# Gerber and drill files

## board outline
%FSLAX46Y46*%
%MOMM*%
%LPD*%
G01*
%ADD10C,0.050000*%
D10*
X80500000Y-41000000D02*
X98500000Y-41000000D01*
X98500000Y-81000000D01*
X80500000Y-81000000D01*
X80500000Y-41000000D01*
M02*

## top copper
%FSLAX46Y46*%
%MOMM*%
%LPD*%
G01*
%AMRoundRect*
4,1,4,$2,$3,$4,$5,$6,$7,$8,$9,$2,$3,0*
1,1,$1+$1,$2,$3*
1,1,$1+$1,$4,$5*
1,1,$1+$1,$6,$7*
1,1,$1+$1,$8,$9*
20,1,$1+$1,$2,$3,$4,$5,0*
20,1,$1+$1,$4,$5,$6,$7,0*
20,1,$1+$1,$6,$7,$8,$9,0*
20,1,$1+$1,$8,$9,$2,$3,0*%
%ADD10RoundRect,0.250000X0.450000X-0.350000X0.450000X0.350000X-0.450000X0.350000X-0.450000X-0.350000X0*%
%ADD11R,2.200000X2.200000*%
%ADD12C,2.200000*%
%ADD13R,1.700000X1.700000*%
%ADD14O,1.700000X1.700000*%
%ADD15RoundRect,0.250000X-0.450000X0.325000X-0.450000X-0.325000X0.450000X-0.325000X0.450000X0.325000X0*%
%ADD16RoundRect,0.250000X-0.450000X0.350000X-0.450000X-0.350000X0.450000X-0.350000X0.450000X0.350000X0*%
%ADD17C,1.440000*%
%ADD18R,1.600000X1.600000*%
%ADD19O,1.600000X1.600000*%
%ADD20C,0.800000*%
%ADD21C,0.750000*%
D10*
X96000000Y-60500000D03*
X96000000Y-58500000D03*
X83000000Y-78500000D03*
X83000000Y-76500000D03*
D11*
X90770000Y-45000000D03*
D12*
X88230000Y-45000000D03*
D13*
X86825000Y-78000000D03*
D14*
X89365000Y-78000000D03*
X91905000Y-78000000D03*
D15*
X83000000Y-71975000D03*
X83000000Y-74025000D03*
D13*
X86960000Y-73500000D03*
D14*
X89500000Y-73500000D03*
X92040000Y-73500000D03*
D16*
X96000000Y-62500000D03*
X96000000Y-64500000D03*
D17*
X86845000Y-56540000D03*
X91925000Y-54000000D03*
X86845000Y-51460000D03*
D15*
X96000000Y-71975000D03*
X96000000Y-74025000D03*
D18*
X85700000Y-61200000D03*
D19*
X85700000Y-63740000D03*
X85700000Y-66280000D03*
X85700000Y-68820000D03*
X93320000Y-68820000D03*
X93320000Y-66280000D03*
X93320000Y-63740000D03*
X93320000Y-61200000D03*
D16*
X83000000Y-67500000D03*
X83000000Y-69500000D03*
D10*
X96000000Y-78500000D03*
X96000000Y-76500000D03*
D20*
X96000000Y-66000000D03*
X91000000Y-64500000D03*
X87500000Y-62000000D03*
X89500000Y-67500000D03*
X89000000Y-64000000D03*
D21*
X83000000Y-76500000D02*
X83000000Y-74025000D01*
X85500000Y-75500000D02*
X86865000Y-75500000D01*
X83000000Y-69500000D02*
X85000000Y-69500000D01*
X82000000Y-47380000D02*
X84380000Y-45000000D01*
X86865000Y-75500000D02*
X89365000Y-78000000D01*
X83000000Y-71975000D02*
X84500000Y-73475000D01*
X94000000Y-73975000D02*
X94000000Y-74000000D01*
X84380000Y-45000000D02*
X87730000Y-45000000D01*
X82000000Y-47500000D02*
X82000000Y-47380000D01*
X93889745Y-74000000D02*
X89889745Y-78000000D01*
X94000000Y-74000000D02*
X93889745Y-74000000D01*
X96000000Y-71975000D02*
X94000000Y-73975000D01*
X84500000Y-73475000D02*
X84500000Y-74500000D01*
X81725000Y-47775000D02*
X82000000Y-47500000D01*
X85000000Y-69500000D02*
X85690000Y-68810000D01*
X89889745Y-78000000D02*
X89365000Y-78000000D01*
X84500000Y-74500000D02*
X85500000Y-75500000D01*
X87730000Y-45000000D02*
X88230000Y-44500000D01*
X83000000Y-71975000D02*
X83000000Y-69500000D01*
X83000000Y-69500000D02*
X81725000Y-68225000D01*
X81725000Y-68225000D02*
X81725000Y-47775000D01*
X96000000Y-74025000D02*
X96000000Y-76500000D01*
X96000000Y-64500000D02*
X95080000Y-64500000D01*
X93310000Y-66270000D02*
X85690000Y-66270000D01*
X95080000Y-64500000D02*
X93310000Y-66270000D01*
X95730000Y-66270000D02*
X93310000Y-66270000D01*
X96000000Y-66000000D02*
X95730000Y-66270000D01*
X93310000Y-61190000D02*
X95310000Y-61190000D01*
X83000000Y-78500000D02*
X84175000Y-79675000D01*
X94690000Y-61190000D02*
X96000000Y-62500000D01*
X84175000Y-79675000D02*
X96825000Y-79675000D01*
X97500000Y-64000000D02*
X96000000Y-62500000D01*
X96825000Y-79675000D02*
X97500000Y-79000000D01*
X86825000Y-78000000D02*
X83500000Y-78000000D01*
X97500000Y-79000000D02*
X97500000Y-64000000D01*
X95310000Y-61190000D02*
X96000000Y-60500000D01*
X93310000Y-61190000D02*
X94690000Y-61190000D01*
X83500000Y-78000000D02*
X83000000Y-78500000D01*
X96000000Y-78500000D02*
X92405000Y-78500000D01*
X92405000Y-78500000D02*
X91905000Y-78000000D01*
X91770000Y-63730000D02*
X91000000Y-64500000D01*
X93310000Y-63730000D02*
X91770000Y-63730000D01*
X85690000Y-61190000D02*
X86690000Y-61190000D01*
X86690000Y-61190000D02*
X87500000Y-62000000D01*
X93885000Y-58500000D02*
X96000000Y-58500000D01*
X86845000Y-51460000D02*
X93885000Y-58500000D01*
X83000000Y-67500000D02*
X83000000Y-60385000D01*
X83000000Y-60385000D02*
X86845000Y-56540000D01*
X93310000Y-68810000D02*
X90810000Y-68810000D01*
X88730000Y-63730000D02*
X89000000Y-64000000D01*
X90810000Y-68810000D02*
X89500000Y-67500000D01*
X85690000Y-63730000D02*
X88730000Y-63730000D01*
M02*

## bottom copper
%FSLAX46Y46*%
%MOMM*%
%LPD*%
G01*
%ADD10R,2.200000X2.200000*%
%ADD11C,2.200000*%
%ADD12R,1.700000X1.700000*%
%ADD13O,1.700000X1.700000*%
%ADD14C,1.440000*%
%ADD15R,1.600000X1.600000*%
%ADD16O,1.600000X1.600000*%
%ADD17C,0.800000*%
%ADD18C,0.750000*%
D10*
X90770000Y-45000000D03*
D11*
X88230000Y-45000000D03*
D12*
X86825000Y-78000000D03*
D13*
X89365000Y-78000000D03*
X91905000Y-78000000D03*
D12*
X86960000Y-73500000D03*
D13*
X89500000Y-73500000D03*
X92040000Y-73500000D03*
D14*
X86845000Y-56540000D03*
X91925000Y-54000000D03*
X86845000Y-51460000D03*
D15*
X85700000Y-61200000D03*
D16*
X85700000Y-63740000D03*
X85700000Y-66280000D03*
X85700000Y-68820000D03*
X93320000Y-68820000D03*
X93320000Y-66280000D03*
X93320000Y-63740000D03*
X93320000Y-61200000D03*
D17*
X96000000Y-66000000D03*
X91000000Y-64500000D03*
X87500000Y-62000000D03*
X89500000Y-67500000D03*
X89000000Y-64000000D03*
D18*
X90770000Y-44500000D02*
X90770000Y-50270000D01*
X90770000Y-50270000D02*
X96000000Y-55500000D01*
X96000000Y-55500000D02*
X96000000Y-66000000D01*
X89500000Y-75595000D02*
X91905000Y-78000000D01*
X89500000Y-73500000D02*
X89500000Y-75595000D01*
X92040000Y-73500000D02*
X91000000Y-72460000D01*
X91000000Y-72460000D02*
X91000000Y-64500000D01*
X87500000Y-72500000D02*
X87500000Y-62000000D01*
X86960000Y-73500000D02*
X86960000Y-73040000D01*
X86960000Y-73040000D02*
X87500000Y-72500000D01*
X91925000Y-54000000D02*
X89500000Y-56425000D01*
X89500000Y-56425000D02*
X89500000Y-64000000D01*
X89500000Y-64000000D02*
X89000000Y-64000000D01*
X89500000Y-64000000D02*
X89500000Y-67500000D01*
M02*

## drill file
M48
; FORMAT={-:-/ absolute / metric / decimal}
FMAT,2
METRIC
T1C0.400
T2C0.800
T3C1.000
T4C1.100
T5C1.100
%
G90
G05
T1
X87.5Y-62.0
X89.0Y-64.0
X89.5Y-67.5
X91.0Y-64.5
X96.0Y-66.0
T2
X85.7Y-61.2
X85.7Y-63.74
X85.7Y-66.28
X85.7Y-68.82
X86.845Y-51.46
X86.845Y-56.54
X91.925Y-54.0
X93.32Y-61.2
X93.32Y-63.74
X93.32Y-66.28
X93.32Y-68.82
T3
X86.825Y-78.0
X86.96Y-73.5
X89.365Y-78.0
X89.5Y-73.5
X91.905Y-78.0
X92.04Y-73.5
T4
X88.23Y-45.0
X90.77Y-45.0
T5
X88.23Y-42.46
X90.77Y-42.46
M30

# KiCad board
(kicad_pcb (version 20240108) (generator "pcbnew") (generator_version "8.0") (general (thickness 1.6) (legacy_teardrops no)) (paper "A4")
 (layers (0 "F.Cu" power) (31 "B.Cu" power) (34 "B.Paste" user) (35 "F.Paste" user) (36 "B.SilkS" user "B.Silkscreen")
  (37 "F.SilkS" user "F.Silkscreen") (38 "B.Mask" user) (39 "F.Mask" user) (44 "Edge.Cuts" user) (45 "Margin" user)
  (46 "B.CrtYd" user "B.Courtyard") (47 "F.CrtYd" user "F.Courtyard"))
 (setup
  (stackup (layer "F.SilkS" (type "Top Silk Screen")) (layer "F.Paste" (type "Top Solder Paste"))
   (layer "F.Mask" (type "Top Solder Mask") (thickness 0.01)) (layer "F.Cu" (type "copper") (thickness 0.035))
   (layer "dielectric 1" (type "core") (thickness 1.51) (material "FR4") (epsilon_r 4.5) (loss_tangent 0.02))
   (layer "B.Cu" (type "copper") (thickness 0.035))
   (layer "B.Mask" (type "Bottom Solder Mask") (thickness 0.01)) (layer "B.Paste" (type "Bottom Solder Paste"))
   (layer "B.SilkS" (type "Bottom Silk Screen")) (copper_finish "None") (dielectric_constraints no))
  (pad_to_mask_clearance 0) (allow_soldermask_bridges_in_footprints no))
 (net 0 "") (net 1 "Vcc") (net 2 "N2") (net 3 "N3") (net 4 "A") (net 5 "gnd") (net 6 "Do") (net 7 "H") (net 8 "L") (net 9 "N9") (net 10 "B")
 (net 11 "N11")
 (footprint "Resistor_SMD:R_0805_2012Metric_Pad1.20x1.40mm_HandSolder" (layer "F.Cu") (at 96 59.5 90)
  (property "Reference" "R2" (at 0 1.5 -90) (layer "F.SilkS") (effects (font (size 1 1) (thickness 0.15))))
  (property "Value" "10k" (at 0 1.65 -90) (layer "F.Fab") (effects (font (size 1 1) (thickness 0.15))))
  (pad "1" smd roundrect (at -1 0 90) (size 1.2 1.4) (layers "F.Cu" "F.Paste" "F.Mask") (roundrect_rratio 0.208333) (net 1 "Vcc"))
  (pad "2" smd roundrect (at 1 0 90) (size 1.2 1.4) (layers "F.Cu" "F.Paste" "F.Mask") (roundrect_rratio 0.208333) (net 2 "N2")))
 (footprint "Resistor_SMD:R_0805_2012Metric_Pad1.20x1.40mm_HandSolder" (layer "F.Cu") (at 83 77.5 90)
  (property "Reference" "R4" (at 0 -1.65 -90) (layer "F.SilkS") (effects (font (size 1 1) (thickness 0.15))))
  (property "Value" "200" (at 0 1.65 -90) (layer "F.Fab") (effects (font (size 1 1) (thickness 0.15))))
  (pad "1" smd roundrect (at -1 0 90) (size 1.2 1.4) (layers "F.Cu" "F.Paste" "F.Mask") (roundrect_rratio 0.208333) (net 1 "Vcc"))
  (pad "2" smd roundrect (at 1 0 90) (size 1.2 1.4) (layers "F.Cu" "F.Paste" "F.Mask") (roundrect_rratio 0.208333) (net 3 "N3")))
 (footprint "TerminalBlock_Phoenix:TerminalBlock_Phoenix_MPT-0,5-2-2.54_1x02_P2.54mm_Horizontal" (layer "F.Cu") (at 90.77 45 180)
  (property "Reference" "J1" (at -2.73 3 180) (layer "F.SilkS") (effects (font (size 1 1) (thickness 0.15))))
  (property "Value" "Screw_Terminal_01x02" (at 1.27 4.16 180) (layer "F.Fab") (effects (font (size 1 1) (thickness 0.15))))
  (pad "" np_thru_hole circle (at 0 2.54 180) (size 1.1 1.1) (drill 1.1) (layers "*.Cu" "*.Mask"))
  (pad "" np_thru_hole circle (at 2.54 2.54 180) (size 1.1 1.1) (drill 1.1) (layers "*.Cu" "*.Mask"))
  (pad "1" thru_hole rect (at 0 0 180) (size 2.2 2.2) (drill 1.1) (layers "*.Cu" "*.Mask") (remove_unused_layers no) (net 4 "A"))
  (pad "2" thru_hole circle (at 2.54 0 180) (size 2.2 2.2) (drill 1.1) (layers "*.Cu" "*.Mask") (remove_unused_layers no) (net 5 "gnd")))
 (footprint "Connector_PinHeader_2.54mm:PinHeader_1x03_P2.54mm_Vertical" (layer "F.Cu") (at 86.825 78 90)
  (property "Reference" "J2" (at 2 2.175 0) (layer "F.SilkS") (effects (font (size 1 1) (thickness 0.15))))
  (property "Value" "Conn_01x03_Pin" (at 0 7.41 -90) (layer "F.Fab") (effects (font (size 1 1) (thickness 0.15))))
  (pad "1" thru_hole rect (at 0 0 90) (size 1.7 1.7) (drill 1) (layers "*.Cu" "*.Mask") (remove_unused_layers no) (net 1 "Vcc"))
  (pad "2" thru_hole oval (at 0 2.54 90) (size 1.7 1.7) (drill 1) (layers "*.Cu" "*.Mask") (remove_unused_layers no) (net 5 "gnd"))
  (pad "3" thru_hole oval (at 0 5.08 90) (size 1.7 1.7) (drill 1) (layers "*.Cu" "*.Mask") (remove_unused_layers no) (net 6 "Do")))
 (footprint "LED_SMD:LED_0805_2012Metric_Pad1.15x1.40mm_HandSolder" (layer "F.Cu") (at 83 73 -90)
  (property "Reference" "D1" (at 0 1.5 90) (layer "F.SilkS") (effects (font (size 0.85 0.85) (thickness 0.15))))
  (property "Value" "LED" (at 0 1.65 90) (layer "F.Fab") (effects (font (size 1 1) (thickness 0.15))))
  (pad "1" smd roundrect (at -1.025 0 270) (size 1.15 1.4) (layers "F.Cu" "F.Paste" "F.Mask") (roundrect_rratio 0.217391) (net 5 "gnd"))
  (pad "2" smd roundrect (at 1.025 0 270) (size 1.15 1.4) (layers "F.Cu" "F.Paste" "F.Mask") (roundrect_rratio 0.217391) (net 3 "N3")))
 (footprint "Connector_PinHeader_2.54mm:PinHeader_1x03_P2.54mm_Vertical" (layer "F.Cu") (at 86.96 73.5 90)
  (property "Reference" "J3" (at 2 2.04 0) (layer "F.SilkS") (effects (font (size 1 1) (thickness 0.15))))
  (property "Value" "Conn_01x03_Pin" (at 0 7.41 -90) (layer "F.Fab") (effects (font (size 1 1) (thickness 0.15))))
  (pad "1" thru_hole rect (at 0 0 90) (size 1.7 1.7) (drill 1) (layers "*.Cu" "*.Mask") (remove_unused_layers no) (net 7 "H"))
  (pad "2" thru_hole oval (at 0 2.54 90) (size 1.7 1.7) (drill 1) (layers "*.Cu" "*.Mask") (remove_unused_layers no) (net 6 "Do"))
  (pad "3" thru_hole oval (at 0 5.08 90) (size 1.7 1.7) (drill 1) (layers "*.Cu" "*.Mask") (remove_unused_layers no) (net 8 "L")))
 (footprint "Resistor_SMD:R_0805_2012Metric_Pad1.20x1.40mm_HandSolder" (layer "F.Cu") (at 96 63.5 -90)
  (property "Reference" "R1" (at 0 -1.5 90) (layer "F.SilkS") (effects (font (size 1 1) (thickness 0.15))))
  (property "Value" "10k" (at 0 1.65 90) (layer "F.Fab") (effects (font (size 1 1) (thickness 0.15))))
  (pad "1" smd roundrect (at -1 0 270) (size 1.2 1.4) (layers "F.Cu" "F.Paste" "F.Mask") (roundrect_rratio 0.208333) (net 1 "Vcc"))
  (pad "2" smd roundrect (at 1 0 270) (size 1.2 1.4) (layers "F.Cu" "F.Paste" "F.Mask") (roundrect_rratio 0.208333) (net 4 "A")))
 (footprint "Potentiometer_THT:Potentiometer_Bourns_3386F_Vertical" (layer "F.Cu") (at 86.845 56.54)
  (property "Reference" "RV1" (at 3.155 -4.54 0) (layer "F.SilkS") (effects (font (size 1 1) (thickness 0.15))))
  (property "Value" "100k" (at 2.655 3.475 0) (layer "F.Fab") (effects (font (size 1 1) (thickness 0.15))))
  (pad "1" thru_hole circle (at 0 0) (size 1.44 1.44) (drill 0.8) (layers "*.Cu" "*.Mask") (remove_unused_layers no) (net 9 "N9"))
  (pad "2" thru_hole circle (at 5.08 -2.54) (size 1.44 1.44) (drill 0.8) (layers "*.Cu" "*.Mask") (remove_unused_layers no) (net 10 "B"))
  (pad "3" thru_hole circle (at 0 -5.08) (size 1.44 1.44) (drill 0.8) (layers "*.Cu" "*.Mask") (remove_unused_layers no) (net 2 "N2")))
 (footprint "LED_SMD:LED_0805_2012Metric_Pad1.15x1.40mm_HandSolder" (layer "F.Cu") (at 96 73 -90)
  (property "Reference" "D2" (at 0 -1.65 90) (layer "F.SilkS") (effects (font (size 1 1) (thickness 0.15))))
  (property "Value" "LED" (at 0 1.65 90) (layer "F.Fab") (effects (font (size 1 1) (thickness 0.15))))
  (pad "1" smd roundrect (at -1.025 0 270) (size 1.15 1.4) (layers "F.Cu" "F.Paste" "F.Mask") (roundrect_rratio 0.217391) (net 5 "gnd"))
  (pad "2" smd roundrect (at 1.025 0 270) (size 1.15 1.4) (layers "F.Cu" "F.Paste" "F.Mask") (roundrect_rratio 0.217391) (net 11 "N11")))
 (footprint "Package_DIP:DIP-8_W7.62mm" (layer "F.Cu") (at 85.7 61.2)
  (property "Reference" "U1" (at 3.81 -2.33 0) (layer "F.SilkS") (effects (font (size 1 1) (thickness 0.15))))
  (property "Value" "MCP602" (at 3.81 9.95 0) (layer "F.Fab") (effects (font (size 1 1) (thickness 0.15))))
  (pad "1" thru_hole rect (at 0 0) (size 1.6 1.6) (drill 0.8) (layers "*.Cu" "*.Mask") (remove_unused_layers no) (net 7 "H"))
  (pad "2" thru_hole oval (at 0 2.54) (size 1.6 1.6) (drill 0.8) (layers "*.Cu" "*.Mask") (remove_unused_layers no) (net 10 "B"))
  (pad "3" thru_hole oval (at 0 5.08) (size 1.6 1.6) (drill 0.8) (layers "*.Cu" "*.Mask") (remove_unused_layers no) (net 4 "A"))
  (pad "4" thru_hole oval (at 0 7.62) (size 1.6 1.6) (drill 0.8) (layers "*.Cu" "*.Mask") (remove_unused_layers no) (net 5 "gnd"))
  (pad "5" thru_hole oval (at 7.62 7.62) (size 1.6 1.6) (drill 0.8) (layers "*.Cu" "*.Mask") (remove_unused_layers no) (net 10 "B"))
  (pad "6" thru_hole oval (at 7.62 5.08) (size 1.6 1.6) (drill 0.8) (layers "*.Cu" "*.Mask") (remove_unused_layers no) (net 4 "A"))
  (pad "7" thru_hole oval (at 7.62 2.54) (size 1.6 1.6) (drill 0.8) (layers "*.Cu" "*.Mask") (remove_unused_layers no) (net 8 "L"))
  (pad "8" thru_hole oval (at 7.62 0) (size 1.6 1.6) (drill 0.8) (layers "*.Cu" "*.Mask") (remove_unused_layers no) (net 1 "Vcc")))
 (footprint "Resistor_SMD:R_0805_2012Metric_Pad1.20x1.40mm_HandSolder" (layer "F.Cu") (at 83 68.5 -90)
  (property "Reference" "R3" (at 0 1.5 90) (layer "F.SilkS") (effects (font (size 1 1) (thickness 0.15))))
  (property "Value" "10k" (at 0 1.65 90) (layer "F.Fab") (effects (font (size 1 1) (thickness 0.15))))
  (pad "1" smd roundrect (at -1 0 270) (size 1.2 1.4) (layers "F.Cu" "F.Paste" "F.Mask") (roundrect_rratio 0.208333) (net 9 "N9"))
  (pad "2" smd roundrect (at 1 0 270) (size 1.2 1.4) (layers "F.Cu" "F.Paste" "F.Mask") (roundrect_rratio 0.208333) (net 5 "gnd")))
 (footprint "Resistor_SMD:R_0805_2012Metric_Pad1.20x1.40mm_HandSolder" (layer "F.Cu") (at 96 77.5 90)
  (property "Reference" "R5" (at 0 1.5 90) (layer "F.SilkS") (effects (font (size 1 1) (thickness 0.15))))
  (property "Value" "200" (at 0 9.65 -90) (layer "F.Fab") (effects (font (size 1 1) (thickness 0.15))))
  (pad "1" smd roundrect (at -1 0 90) (size 1.2 1.4) (layers "F.Cu" "F.Paste" "F.Mask") (roundrect_rratio 0.208333) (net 6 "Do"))
  (pad "2" smd roundrect (at 1 0 90) (size 1.2 1.4) (layers "F.Cu" "F.Paste" "F.Mask") (roundrect_rratio 0.208333) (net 11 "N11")))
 (gr_rect (start 80.5 41) (end 98.5 81) (stroke (width 0.05) (type default)) (fill none) (layer "Edge.Cuts"))
 (segment (start 83 76.5) (end 83 74.025) (width 0.75) (layer "F.Cu") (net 3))
 (segment (start 85.5 75.5) (end 86.865 75.5) (width 0.75) (layer "F.Cu") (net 5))
 (segment (start 83 69.5) (end 85 69.5) (width 0.75) (layer "F.Cu") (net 5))
 (segment (start 82 47.38) (end 84.38 45) (width 0.75) (layer "F.Cu") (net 5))
 (segment (start 86.865 75.5) (end 89.365 78) (width 0.75) (layer "F.Cu") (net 5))
 (segment (start 83 71.975) (end 84.5 73.475) (width 0.75) (layer "F.Cu") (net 5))
 (segment (start 94 73.975) (end 94 74) (width 0.75) (layer "F.Cu") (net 5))
 (segment (start 84.38 45) (end 87.73 45) (width 0.75) (layer "F.Cu") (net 5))
 (segment (start 82 47.5) (end 82 47.38) (width 0.75) (layer "F.Cu") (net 5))
 (segment (start 93.889745 74) (end 89.889745 78) (width 0.75) (layer "F.Cu") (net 5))
 (segment (start 94 74) (end 93.889745 74) (width 0.75) (layer "F.Cu") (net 5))
 (segment (start 96 71.975) (end 94 73.975) (width 0.75) (layer "F.Cu") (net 5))
 (segment (start 84.5 73.475) (end 84.5 74.5) (width 0.75) (layer "F.Cu") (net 5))
 (segment (start 81.725 47.775) (end 82 47.5) (width 0.75) (layer "F.Cu") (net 5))
 (segment (start 85 69.5) (end 85.69 68.81) (width 0.75) (layer "F.Cu") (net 5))
 (segment (start 89.889745 78) (end 89.365 78) (width 0.75) (layer "F.Cu") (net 5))
 (segment (start 84.5 74.5) (end 85.5 75.5) (width 0.75) (layer "F.Cu") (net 5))
 (segment (start 87.73 45) (end 88.23 44.5) (width 0.75) (layer "F.Cu") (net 5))
 (segment (start 83 71.975) (end 83 69.5) (width 0.75) (layer "F.Cu") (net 5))
 (segment (start 83 69.5) (end 81.725 68.225) (width 0.75) (layer "F.Cu") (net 5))
 (segment (start 81.725 68.225) (end 81.725 47.775) (width 0.75) (layer "F.Cu") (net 5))
 (segment (start 96 74.025) (end 96 76.5) (width 0.75) (layer "F.Cu") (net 11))
 (segment (start 96 64.5) (end 95.08 64.5) (width 0.75) (layer "F.Cu") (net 4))
 (segment (start 93.31 66.27) (end 85.69 66.27) (width 0.75) (layer "F.Cu") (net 4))
 (segment (start 95.08 64.5) (end 93.31 66.27) (width 0.75) (layer "F.Cu") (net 4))
 (segment (start 95.73 66.27) (end 93.31 66.27) (width 0.75) (layer "F.Cu") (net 4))
 (segment (start 96 66) (end 95.73 66.27) (width 0.75) (layer "F.Cu") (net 4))
 (via (at 96 66) (size 0.8) (drill 0.4) (layers "F.Cu" "B.Cu") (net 4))
 (segment (start 90.77 44.5) (end 90.77 50.27) (width 0.75) (layer "B.Cu") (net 4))
 (segment (start 90.77 50.27) (end 96 55.5) (width 0.75) (layer "B.Cu") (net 4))
 (segment (start 96 55.5) (end 96 66) (width 0.75) (layer "B.Cu") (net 4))
 (segment (start 93.31 61.19) (end 95.31 61.19) (width 0.75) (layer "F.Cu") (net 1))
 (segment (start 83 78.5) (end 84.175 79.675) (width 0.75) (layer "F.Cu") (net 1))
 (segment (start 94.69 61.19) (end 96 62.5) (width 0.75) (layer "F.Cu") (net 1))
 (segment (start 84.175 79.675) (end 96.825 79.675) (width 0.75) (layer "F.Cu") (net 1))
 (segment (start 97.5 64) (end 96 62.5) (width 0.75) (layer "F.Cu") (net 1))
 (segment (start 96.825 79.675) (end 97.5 79) (width 0.75) (layer "F.Cu") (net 1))
 (segment (start 86.825 78) (end 83.5 78) (width 0.75) (layer "F.Cu") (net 1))
 (segment (start 97.5 79) (end 97.5 64) (width 0.75) (layer "F.Cu") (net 1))
 (segment (start 95.31 61.19) (end 96 60.5) (width 0.75) (layer "F.Cu") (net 1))
 (segment (start 93.31 61.19) (end 94.69 61.19) (width 0.75) (layer "F.Cu") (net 1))
 (segment (start 83.5 78) (end 83 78.5) (width 0.75) (layer "F.Cu") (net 1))
 (segment (start 96 78.5) (end 92.405 78.5) (width 0.75) (layer "F.Cu") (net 6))
 (segment (start 92.405 78.5) (end 91.905 78) (width 0.75) (layer "F.Cu") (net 6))
 (segment (start 89.5 75.595) (end 91.905 78) (width 0.75) (layer "B.Cu") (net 6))
 (segment (start 89.5 73.5) (end 89.5 75.595) (width 0.75) (layer "B.Cu") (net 6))
 (segment (start 91.77 63.73) (end 91 64.5) (width 0.75) (layer "F.Cu") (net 8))
 (segment (start 93.31 63.73) (end 91.77 63.73) (width 0.75) (layer "F.Cu") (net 8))
 (via (at 91 64.5) (size 0.8) (drill 0.4) (layers "F.Cu" "B.Cu") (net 8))
 (segment (start 92.04 73.5) (end 91 72.46) (width 0.75) (layer "B.Cu") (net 8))
 (segment (start 91 72.46) (end 91 64.5) (width 0.75) (layer "B.Cu") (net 8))
 (segment (start 85.69 61.19) (end 86.69 61.19) (width 0.75) (layer "F.Cu") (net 7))
 (segment (start 86.69 61.19) (end 87.5 62) (width 0.75) (layer "F.Cu") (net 7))
 (via (at 87.5 62) (size 0.8) (drill 0.4) (layers "F.Cu" "B.Cu") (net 7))
 (segment (start 87.5 72.5) (end 87.5 62) (width 0.75) (layer "B.Cu") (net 7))
 (segment (start 86.96 73.5) (end 86.96 73.04) (width 0.75) (layer "B.Cu") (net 7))
 (segment (start 86.96 73.04) (end 87.5 72.5) (width 0.75) (layer "B.Cu") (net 7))
 (segment (start 93.885 58.5) (end 96 58.5) (width 0.75) (layer "F.Cu") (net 2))
 (segment (start 86.845 51.46) (end 93.885 58.5) (width 0.75) (layer "F.Cu") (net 2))
 (segment (start 83 67.5) (end 83 60.385) (width 0.75) (layer "F.Cu") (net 9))
 (segment (start 83 60.385) (end 86.845 56.54) (width 0.75) (layer "F.Cu") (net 9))
 (segment (start 93.31 68.81) (end 90.81 68.81) (width 0.75) (layer "F.Cu") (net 10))
 (segment (start 88.73 63.73) (end 89 64) (width 0.75) (layer "F.Cu") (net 10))
 (segment (start 90.81 68.81) (end 89.5 67.5) (width 0.75) (layer "F.Cu") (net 10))
 (segment (start 85.69 63.73) (end 88.73 63.73) (width 0.75) (layer "F.Cu") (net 10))
 (via (at 89.5 67.5) (size 0.8) (drill 0.4) (layers "F.Cu" "B.Cu") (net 10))
 (via (at 89 64) (size 0.8) (drill 0.4) (layers "F.Cu" "B.Cu") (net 10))
 (segment (start 91.925 54) (end 89.5 56.425) (width 0.75) (layer "B.Cu") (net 10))
 (segment (start 89.5 56.425) (end 89.5 64) (width 0.75) (layer "B.Cu") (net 10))
 (segment (start 89.5 64) (end 89 64) (width 0.75) (layer "B.Cu") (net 10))
 (segment (start 89.5 64) (end 89.5 67.5) (width 0.75) (layer "B.Cu") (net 10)))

